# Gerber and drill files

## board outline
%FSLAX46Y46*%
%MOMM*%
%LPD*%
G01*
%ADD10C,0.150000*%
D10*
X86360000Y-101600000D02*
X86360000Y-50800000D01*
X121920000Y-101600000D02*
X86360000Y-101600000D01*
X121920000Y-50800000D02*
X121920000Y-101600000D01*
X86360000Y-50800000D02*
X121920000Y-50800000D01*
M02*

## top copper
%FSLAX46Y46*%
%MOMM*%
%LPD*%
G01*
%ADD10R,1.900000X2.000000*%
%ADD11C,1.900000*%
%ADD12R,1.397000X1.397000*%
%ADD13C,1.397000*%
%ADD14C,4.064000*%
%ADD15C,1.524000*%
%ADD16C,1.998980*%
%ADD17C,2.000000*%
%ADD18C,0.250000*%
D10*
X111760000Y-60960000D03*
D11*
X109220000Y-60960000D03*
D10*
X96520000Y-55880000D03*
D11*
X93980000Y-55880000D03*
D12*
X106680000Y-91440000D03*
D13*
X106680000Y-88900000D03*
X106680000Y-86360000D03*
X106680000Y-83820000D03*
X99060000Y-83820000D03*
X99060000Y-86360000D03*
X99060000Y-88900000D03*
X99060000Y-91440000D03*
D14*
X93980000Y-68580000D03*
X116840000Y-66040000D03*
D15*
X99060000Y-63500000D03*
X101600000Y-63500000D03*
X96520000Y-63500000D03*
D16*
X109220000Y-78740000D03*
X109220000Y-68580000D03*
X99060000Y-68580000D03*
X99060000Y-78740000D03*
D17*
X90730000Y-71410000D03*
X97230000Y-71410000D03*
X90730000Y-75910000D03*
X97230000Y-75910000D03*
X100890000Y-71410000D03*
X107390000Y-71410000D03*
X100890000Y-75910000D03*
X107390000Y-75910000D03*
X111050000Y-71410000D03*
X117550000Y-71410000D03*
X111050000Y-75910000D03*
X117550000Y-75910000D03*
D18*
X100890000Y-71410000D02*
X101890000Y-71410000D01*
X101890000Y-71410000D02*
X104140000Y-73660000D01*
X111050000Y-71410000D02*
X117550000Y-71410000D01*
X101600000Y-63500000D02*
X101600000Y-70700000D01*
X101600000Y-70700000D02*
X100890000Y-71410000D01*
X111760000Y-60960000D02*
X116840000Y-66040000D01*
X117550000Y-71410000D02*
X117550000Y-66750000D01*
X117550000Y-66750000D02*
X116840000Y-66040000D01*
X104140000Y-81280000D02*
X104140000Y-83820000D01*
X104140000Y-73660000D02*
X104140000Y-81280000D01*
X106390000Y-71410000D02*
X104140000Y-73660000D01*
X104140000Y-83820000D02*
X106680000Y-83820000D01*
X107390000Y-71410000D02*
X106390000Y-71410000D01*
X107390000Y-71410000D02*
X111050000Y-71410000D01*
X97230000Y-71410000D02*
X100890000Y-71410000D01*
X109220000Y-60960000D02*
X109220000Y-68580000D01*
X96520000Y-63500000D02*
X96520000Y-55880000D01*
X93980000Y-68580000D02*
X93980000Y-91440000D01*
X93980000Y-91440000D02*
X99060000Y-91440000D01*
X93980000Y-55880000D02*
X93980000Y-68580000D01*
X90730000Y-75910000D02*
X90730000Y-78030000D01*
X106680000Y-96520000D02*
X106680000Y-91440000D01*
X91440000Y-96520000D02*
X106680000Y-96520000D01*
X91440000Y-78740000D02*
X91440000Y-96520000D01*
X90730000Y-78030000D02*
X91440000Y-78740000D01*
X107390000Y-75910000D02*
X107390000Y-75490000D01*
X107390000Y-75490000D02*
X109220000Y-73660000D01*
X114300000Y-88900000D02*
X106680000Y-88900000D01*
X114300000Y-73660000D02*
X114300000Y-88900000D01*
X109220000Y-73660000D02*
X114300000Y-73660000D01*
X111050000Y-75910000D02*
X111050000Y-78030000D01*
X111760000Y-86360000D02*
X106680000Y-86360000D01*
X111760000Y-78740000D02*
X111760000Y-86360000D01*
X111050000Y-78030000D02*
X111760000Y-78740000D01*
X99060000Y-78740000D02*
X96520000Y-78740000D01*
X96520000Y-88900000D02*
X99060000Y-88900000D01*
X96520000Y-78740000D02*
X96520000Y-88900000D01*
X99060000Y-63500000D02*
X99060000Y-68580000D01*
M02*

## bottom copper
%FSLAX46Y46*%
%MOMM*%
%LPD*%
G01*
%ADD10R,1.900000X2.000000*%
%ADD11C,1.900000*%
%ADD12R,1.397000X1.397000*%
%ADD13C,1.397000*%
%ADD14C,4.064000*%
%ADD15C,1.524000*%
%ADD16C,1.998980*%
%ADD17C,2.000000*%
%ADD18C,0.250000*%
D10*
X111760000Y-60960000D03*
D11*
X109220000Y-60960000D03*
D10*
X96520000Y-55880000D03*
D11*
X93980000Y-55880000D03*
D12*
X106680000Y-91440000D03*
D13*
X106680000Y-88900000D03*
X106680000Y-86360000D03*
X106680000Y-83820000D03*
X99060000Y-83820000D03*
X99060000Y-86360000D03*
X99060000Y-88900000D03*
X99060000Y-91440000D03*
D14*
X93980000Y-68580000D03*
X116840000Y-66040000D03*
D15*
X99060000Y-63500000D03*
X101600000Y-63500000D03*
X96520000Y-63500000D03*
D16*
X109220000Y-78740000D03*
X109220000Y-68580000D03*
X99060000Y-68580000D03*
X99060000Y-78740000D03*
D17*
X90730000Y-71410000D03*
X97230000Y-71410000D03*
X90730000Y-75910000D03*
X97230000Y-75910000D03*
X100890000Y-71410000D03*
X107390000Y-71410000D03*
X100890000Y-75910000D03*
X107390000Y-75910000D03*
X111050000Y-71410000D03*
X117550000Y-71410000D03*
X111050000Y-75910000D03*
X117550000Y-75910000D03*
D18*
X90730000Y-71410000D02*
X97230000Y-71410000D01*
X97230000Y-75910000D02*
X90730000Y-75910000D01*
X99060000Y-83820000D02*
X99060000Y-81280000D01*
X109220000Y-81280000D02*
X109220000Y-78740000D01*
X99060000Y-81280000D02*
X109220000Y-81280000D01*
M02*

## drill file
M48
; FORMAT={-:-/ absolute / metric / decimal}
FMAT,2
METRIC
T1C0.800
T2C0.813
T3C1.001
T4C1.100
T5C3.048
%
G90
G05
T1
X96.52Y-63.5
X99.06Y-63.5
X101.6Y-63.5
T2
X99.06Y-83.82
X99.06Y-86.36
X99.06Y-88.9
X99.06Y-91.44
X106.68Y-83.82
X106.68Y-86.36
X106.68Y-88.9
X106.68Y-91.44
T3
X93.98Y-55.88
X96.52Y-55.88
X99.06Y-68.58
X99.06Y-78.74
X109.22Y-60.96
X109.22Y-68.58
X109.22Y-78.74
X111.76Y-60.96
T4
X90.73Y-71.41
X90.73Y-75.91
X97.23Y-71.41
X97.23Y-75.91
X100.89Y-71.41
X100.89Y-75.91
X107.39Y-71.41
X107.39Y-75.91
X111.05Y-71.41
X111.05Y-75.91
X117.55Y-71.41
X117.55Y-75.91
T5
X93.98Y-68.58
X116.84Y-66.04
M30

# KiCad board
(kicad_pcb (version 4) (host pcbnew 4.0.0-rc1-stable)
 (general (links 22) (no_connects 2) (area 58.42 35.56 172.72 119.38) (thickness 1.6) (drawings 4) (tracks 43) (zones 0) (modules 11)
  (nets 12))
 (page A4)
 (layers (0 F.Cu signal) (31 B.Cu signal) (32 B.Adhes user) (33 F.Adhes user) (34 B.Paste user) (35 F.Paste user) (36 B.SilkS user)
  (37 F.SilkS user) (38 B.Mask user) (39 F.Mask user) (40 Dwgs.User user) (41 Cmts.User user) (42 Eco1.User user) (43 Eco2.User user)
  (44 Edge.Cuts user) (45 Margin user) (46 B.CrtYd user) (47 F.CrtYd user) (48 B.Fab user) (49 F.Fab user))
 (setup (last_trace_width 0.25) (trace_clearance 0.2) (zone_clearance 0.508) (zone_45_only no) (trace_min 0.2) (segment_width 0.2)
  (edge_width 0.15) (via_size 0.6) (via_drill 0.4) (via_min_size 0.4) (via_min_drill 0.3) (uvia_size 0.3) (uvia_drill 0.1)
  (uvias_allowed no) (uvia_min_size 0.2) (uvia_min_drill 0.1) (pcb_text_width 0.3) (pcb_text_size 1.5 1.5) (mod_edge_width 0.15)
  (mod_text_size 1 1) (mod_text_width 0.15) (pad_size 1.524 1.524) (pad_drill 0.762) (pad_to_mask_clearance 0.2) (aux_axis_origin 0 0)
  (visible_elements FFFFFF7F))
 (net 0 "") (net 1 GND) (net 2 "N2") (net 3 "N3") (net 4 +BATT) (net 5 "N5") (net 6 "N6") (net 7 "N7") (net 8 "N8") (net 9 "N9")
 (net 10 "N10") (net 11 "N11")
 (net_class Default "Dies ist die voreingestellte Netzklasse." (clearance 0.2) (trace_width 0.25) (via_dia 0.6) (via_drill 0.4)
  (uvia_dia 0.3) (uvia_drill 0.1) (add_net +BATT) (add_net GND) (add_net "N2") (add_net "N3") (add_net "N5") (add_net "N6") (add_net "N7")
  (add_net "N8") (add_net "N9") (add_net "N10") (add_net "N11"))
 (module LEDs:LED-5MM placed (layer F.Cu) (at 111.76 60.96 180)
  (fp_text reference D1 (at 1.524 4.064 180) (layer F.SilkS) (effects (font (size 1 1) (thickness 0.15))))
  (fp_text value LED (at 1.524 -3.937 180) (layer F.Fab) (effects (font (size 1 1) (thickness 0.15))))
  (pad 1 thru_hole rect (at 0 0 270) (size 2 1.9) (drill 1.00076) (layers *.Cu *.Mask F.SilkS) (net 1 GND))
  (pad 2 thru_hole circle (at 2.54 0 180) (size 1.9 1.9) (drill 1.00076) (layers *.Cu *.Mask F.SilkS) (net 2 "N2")))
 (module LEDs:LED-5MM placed (layer F.Cu) (at 96.52 55.88 180)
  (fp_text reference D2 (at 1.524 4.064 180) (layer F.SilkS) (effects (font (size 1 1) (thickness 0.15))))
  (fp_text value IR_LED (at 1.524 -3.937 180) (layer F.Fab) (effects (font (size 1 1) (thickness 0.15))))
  (pad 1 thru_hole rect (at 0 0 270) (size 2 1.9) (drill 1.00076) (layers *.Cu *.Mask F.SilkS) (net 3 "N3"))
  (pad 2 thru_hole circle (at 2.54 0 180) (size 1.9 1.9) (drill 1.00076) (layers *.Cu *.Mask F.SilkS) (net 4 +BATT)))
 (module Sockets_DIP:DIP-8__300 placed (layer F.Cu) (at 102.87 87.63 90)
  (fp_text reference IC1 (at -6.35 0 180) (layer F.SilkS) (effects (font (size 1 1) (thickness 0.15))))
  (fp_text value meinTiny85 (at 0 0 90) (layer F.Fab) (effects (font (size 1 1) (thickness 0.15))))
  (pad 1 thru_hole rect (at -3.81 3.81 90) (size 1.397 1.397) (drill 0.8128) (layers *.Cu *.Mask F.SilkS) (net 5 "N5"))
  (pad 2 thru_hole circle (at -1.27 3.81 90) (size 1.397 1.397) (drill 0.8128) (layers *.Cu *.Mask F.SilkS) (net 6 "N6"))
  (pad 3 thru_hole circle (at 1.27 3.81 90) (size 1.397 1.397) (drill 0.8128) (layers *.Cu *.Mask F.SilkS) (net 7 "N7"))
  (pad 4 thru_hole circle (at 3.81 3.81 90) (size 1.397 1.397) (drill 0.8128) (layers *.Cu *.Mask F.SilkS) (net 1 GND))
  (pad 5 thru_hole circle (at 3.81 -3.81 90) (size 1.397 1.397) (drill 0.8128) (layers *.Cu *.Mask F.SilkS) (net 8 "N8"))
  (pad 6 thru_hole circle (at 1.27 -3.81 90) (size 1.397 1.397) (drill 0.8128) (layers *.Cu *.Mask F.SilkS) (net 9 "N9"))
  (pad 7 thru_hole circle (at -1.27 -3.81 90) (size 1.397 1.397) (drill 0.8128) (layers *.Cu *.Mask F.SilkS) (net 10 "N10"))
  (pad 8 thru_hole circle (at -3.81 -3.81 90) (size 1.397 1.397) (drill 0.8128) (layers *.Cu *.Mask F.SilkS) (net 4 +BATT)))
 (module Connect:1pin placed (layer F.Cu) (at 93.98 68.58)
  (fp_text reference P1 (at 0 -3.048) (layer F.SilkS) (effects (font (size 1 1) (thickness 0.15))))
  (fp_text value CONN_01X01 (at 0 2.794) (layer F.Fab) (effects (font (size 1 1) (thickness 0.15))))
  (pad 1 thru_hole circle (at 0 0) (size 4.064 4.064) (drill 3.048) (layers *.Cu *.Mask F.SilkS) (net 4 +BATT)))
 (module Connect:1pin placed (layer F.Cu) (at 116.84 66.04)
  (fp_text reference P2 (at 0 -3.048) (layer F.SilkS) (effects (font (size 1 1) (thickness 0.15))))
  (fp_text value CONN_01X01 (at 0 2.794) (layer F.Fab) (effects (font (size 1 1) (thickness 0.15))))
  (pad 1 thru_hole circle (at 0 0) (size 4.064 4.064) (drill 3.048) (layers *.Cu *.Mask F.SilkS) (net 1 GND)))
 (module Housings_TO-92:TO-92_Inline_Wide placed (layer F.Cu) (at 96.52 63.5)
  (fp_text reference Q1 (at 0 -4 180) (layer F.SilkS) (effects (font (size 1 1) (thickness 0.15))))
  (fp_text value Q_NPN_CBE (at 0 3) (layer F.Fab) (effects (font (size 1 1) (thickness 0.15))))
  (pad 2 thru_hole circle (at 2.54 0 90) (size 1.524 1.524) (drill 0.8) (layers *.Cu *.Mask F.SilkS) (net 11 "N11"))
  (pad 3 thru_hole circle (at 5.08 0 90) (size 1.524 1.524) (drill 0.8) (layers *.Cu *.Mask F.SilkS) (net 1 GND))
  (pad 1 thru_hole circle (at 0 0 90) (size 1.524 1.524) (drill 0.8) (layers *.Cu *.Mask F.SilkS) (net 3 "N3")))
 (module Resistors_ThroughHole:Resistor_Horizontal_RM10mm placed (layer F.Cu) (at 109.22 73.66 90)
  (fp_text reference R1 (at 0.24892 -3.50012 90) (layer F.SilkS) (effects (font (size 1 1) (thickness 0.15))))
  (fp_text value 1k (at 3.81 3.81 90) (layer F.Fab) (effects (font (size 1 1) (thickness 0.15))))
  (pad 1 thru_hole circle (at -5.08 0 90) (size 1.99898 1.99898) (drill 1.00076) (layers *.Cu *.SilkS *.Mask) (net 8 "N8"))
  (pad 2 thru_hole circle (at 5.08 0 90) (size 1.99898 1.99898) (drill 1.00076) (layers *.Cu *.SilkS *.Mask) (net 2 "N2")))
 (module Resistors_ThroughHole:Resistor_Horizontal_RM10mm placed (layer F.Cu) (at 99.06 73.66 270)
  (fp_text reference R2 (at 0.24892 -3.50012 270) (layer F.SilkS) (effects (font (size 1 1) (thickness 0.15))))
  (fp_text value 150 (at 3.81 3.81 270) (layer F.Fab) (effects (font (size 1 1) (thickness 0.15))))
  (pad 1 thru_hole circle (at -5.08 0 270) (size 1.99898 1.99898) (drill 1.00076) (layers *.Cu *.SilkS *.Mask) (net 11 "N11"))
  (pad 2 thru_hole circle (at 5.08 0 270) (size 1.99898 1.99898) (drill 1.00076) (layers *.Cu *.SilkS *.Mask) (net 10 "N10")))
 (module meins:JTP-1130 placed (layer F.Cu) (at 93.98 73.66 180)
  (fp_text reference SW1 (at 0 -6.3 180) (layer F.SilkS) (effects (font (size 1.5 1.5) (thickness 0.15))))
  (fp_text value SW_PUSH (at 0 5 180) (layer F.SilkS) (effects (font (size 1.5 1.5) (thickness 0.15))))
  (pad 1 thru_hole circle (at 3.25 2.25 180) (size 2 2) (drill 1.1) (layers *.Cu *.Mask F.SilkS) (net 1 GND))
  (pad 1 thru_hole circle (at -3.25 2.25 180) (size 2 2) (drill 1.1) (layers *.Cu *.Mask F.SilkS) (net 1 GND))
  (pad 2 thru_hole circle (at 3.25 -2.25 180) (size 2 2) (drill 1.1) (layers *.Cu *.Mask F.SilkS) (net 5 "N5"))
  (pad 2 thru_hole circle (at -3.25 -2.25 180) (size 2 2) (drill 1.1) (layers *.Cu *.Mask F.SilkS) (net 5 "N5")))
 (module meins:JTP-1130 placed (layer F.Cu) (at 104.14 73.66 180)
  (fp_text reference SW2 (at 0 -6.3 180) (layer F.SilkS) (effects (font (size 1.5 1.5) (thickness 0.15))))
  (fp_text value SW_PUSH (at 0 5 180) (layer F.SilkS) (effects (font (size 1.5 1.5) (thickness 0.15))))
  (pad 1 thru_hole circle (at 3.25 2.25 180) (size 2 2) (drill 1.1) (layers *.Cu *.Mask F.SilkS) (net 1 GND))
  (pad 1 thru_hole circle (at -3.25 2.25 180) (size 2 2) (drill 1.1) (layers *.Cu *.Mask F.SilkS) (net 1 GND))
  (pad 2 thru_hole circle (at 3.25 -2.25 180) (size 2 2) (drill 1.1) (layers *.Cu *.Mask F.SilkS) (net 6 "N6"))
  (pad 2 thru_hole circle (at -3.25 -2.25 180) (size 2 2) (drill 1.1) (layers *.Cu *.Mask F.SilkS) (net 6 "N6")))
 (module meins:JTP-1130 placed (layer F.Cu) (at 114.3 73.66 180)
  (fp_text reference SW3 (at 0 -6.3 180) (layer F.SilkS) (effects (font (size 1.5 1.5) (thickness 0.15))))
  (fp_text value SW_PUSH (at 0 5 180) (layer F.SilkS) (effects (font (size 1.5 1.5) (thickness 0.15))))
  (pad 1 thru_hole circle (at 3.25 2.25 180) (size 2 2) (drill 1.1) (layers *.Cu *.Mask F.SilkS) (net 1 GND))
  (pad 1 thru_hole circle (at -3.25 2.25 180) (size 2 2) (drill 1.1) (layers *.Cu *.Mask F.SilkS) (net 1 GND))
  (pad 2 thru_hole circle (at 3.25 -2.25 180) (size 2 2) (drill 1.1) (layers *.Cu *.Mask F.SilkS) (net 7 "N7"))
  (pad 2 thru_hole circle (at -3.25 -2.25 180) (size 2 2) (drill 1.1) (layers *.Cu *.Mask F.SilkS) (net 7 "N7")))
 (gr_line (start 86.36 101.6) (end 86.36 50.8) (angle 90) (layer Edge.Cuts) (width 0.15))
 (gr_line (start 121.92 101.6) (end 86.36 101.6) (angle 90) (layer Edge.Cuts) (width 0.15))
 (gr_line (start 121.92 50.8) (end 121.92 101.6) (angle 90) (layer Edge.Cuts) (width 0.15))
 (gr_line (start 86.36 50.8) (end 121.92 50.8) (angle 90) (layer Edge.Cuts) (width 0.15))
 (segment (start 90.73 71.41) (end 97.23 71.41) (width 0.25) (layer B.Cu) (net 1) (status C00000))
 (segment (start 100.89 71.41) (end 101.89 71.41) (width 0.25) (layer F.Cu) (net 1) (status C00000))
 (segment (start 101.89 71.41) (end 104.14 73.66) (width 0.25) (layer F.Cu) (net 1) (status 400000))
 (segment (start 111.05 71.41) (end 117.55 71.41) (width 0.25) (layer F.Cu) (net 1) (status C00000))
 (segment (start 101.6 63.5) (end 101.6 70.7) (width 0.25) (layer F.Cu) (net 1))
 (segment (start 101.6 70.7) (end 100.89 71.41) (width 0.25) (layer F.Cu) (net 1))
 (segment (start 111.76 60.96) (end 116.84 66.04) (width 0.25) (layer F.Cu) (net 1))
 (segment (start 117.55 71.41) (end 117.55 66.75) (width 0.25) (layer F.Cu) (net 1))
 (segment (start 117.55 66.75) (end 116.84 66.04) (width 0.25) (layer F.Cu) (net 1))
 (segment (start 104.14 81.28) (end 104.14 83.82) (width 0.25) (layer F.Cu) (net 1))
 (segment (start 104.14 73.66) (end 104.14 81.28) (width 0.25) (layer F.Cu) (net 1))
 (segment (start 106.39 71.41) (end 104.14 73.66) (width 0.25) (layer F.Cu) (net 1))
 (segment (start 104.14 83.82) (end 106.68 83.82) (width 0.25) (layer F.Cu) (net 1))
 (segment (start 107.39 71.41) (end 106.39 71.41) (width 0.25) (layer F.Cu) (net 1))
 (segment (start 107.39 71.41) (end 111.05 71.41) (width 0.25) (layer F.Cu) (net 1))
 (segment (start 97.23 71.41) (end 100.89 71.41) (width 0.25) (layer F.Cu) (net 1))
 (segment (start 109.22 60.96) (end 109.22 68.58) (width 0.25) (layer F.Cu) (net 2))
 (segment (start 96.52 63.5) (end 96.52 55.88) (width 0.25) (layer F.Cu) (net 3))
 (segment (start 93.98 68.58) (end 93.98 91.44) (width 0.25) (layer F.Cu) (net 4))
 (segment (start 93.98 91.44) (end 99.06 91.44) (width 0.25) (layer F.Cu) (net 4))
 (segment (start 93.98 55.88) (end 93.98 68.58) (width 0.25) (layer F.Cu) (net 4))
 (segment (start 97.23 75.91) (end 90.73 75.91) (width 0.25) (layer B.Cu) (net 5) (status C00000))
 (segment (start 90.73 75.91) (end 90.73 78.03) (width 0.25) (layer F.Cu) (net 5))
 (segment (start 106.68 96.52) (end 106.68 91.44) (width 0.25) (layer F.Cu) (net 5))
 (segment (start 91.44 96.52) (end 106.68 96.52) (width 0.25) (layer F.Cu) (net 5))
 (segment (start 91.44 78.74) (end 91.44 96.52) (width 0.25) (layer F.Cu) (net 5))
 (segment (start 90.73 78.03) (end 91.44 78.74) (width 0.25) (layer F.Cu) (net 5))
 (segment (start 107.39 75.91) (end 107.39 75.49) (width 0.25) (layer F.Cu) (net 6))
 (segment (start 107.39 75.49) (end 109.22 73.66) (width 0.25) (layer F.Cu) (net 6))
 (segment (start 114.3 88.9) (end 106.68 88.9) (width 0.25) (layer F.Cu) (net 6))
 (segment (start 114.3 73.66) (end 114.3 88.9) (width 0.25) (layer F.Cu) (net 6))
 (segment (start 109.22 73.66) (end 114.3 73.66) (width 0.25) (layer F.Cu) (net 6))
 (segment (start 111.05 75.91) (end 111.05 78.03) (width 0.25) (layer F.Cu) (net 7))
 (segment (start 111.76 86.36) (end 106.68 86.36) (width 0.25) (layer F.Cu) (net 7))
 (segment (start 111.76 78.74) (end 111.76 86.36) (width 0.25) (layer F.Cu) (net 7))
 (segment (start 111.05 78.03) (end 111.76 78.74) (width 0.25) (layer F.Cu) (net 7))
 (segment (start 99.06 83.82) (end 99.06 81.28) (width 0.25) (layer B.Cu) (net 8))
 (segment (start 109.22 81.28) (end 109.22 78.74) (width 0.25) (layer B.Cu) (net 8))
 (segment (start 99.06 81.28) (end 109.22 81.28) (width 0.25) (layer B.Cu) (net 8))
 (segment (start 99.06 78.74) (end 96.52 78.74) (width 0.25) (layer F.Cu) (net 10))
 (segment (start 96.52 88.9) (end 99.06 88.9) (width 0.25) (layer F.Cu) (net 10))
 (segment (start 96.52 78.74) (end 96.52 88.9) (width 0.25) (layer F.Cu) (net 10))
 (segment (start 99.06 63.5) (end 99.06 68.58) (width 0.25) (layer F.Cu) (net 11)))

